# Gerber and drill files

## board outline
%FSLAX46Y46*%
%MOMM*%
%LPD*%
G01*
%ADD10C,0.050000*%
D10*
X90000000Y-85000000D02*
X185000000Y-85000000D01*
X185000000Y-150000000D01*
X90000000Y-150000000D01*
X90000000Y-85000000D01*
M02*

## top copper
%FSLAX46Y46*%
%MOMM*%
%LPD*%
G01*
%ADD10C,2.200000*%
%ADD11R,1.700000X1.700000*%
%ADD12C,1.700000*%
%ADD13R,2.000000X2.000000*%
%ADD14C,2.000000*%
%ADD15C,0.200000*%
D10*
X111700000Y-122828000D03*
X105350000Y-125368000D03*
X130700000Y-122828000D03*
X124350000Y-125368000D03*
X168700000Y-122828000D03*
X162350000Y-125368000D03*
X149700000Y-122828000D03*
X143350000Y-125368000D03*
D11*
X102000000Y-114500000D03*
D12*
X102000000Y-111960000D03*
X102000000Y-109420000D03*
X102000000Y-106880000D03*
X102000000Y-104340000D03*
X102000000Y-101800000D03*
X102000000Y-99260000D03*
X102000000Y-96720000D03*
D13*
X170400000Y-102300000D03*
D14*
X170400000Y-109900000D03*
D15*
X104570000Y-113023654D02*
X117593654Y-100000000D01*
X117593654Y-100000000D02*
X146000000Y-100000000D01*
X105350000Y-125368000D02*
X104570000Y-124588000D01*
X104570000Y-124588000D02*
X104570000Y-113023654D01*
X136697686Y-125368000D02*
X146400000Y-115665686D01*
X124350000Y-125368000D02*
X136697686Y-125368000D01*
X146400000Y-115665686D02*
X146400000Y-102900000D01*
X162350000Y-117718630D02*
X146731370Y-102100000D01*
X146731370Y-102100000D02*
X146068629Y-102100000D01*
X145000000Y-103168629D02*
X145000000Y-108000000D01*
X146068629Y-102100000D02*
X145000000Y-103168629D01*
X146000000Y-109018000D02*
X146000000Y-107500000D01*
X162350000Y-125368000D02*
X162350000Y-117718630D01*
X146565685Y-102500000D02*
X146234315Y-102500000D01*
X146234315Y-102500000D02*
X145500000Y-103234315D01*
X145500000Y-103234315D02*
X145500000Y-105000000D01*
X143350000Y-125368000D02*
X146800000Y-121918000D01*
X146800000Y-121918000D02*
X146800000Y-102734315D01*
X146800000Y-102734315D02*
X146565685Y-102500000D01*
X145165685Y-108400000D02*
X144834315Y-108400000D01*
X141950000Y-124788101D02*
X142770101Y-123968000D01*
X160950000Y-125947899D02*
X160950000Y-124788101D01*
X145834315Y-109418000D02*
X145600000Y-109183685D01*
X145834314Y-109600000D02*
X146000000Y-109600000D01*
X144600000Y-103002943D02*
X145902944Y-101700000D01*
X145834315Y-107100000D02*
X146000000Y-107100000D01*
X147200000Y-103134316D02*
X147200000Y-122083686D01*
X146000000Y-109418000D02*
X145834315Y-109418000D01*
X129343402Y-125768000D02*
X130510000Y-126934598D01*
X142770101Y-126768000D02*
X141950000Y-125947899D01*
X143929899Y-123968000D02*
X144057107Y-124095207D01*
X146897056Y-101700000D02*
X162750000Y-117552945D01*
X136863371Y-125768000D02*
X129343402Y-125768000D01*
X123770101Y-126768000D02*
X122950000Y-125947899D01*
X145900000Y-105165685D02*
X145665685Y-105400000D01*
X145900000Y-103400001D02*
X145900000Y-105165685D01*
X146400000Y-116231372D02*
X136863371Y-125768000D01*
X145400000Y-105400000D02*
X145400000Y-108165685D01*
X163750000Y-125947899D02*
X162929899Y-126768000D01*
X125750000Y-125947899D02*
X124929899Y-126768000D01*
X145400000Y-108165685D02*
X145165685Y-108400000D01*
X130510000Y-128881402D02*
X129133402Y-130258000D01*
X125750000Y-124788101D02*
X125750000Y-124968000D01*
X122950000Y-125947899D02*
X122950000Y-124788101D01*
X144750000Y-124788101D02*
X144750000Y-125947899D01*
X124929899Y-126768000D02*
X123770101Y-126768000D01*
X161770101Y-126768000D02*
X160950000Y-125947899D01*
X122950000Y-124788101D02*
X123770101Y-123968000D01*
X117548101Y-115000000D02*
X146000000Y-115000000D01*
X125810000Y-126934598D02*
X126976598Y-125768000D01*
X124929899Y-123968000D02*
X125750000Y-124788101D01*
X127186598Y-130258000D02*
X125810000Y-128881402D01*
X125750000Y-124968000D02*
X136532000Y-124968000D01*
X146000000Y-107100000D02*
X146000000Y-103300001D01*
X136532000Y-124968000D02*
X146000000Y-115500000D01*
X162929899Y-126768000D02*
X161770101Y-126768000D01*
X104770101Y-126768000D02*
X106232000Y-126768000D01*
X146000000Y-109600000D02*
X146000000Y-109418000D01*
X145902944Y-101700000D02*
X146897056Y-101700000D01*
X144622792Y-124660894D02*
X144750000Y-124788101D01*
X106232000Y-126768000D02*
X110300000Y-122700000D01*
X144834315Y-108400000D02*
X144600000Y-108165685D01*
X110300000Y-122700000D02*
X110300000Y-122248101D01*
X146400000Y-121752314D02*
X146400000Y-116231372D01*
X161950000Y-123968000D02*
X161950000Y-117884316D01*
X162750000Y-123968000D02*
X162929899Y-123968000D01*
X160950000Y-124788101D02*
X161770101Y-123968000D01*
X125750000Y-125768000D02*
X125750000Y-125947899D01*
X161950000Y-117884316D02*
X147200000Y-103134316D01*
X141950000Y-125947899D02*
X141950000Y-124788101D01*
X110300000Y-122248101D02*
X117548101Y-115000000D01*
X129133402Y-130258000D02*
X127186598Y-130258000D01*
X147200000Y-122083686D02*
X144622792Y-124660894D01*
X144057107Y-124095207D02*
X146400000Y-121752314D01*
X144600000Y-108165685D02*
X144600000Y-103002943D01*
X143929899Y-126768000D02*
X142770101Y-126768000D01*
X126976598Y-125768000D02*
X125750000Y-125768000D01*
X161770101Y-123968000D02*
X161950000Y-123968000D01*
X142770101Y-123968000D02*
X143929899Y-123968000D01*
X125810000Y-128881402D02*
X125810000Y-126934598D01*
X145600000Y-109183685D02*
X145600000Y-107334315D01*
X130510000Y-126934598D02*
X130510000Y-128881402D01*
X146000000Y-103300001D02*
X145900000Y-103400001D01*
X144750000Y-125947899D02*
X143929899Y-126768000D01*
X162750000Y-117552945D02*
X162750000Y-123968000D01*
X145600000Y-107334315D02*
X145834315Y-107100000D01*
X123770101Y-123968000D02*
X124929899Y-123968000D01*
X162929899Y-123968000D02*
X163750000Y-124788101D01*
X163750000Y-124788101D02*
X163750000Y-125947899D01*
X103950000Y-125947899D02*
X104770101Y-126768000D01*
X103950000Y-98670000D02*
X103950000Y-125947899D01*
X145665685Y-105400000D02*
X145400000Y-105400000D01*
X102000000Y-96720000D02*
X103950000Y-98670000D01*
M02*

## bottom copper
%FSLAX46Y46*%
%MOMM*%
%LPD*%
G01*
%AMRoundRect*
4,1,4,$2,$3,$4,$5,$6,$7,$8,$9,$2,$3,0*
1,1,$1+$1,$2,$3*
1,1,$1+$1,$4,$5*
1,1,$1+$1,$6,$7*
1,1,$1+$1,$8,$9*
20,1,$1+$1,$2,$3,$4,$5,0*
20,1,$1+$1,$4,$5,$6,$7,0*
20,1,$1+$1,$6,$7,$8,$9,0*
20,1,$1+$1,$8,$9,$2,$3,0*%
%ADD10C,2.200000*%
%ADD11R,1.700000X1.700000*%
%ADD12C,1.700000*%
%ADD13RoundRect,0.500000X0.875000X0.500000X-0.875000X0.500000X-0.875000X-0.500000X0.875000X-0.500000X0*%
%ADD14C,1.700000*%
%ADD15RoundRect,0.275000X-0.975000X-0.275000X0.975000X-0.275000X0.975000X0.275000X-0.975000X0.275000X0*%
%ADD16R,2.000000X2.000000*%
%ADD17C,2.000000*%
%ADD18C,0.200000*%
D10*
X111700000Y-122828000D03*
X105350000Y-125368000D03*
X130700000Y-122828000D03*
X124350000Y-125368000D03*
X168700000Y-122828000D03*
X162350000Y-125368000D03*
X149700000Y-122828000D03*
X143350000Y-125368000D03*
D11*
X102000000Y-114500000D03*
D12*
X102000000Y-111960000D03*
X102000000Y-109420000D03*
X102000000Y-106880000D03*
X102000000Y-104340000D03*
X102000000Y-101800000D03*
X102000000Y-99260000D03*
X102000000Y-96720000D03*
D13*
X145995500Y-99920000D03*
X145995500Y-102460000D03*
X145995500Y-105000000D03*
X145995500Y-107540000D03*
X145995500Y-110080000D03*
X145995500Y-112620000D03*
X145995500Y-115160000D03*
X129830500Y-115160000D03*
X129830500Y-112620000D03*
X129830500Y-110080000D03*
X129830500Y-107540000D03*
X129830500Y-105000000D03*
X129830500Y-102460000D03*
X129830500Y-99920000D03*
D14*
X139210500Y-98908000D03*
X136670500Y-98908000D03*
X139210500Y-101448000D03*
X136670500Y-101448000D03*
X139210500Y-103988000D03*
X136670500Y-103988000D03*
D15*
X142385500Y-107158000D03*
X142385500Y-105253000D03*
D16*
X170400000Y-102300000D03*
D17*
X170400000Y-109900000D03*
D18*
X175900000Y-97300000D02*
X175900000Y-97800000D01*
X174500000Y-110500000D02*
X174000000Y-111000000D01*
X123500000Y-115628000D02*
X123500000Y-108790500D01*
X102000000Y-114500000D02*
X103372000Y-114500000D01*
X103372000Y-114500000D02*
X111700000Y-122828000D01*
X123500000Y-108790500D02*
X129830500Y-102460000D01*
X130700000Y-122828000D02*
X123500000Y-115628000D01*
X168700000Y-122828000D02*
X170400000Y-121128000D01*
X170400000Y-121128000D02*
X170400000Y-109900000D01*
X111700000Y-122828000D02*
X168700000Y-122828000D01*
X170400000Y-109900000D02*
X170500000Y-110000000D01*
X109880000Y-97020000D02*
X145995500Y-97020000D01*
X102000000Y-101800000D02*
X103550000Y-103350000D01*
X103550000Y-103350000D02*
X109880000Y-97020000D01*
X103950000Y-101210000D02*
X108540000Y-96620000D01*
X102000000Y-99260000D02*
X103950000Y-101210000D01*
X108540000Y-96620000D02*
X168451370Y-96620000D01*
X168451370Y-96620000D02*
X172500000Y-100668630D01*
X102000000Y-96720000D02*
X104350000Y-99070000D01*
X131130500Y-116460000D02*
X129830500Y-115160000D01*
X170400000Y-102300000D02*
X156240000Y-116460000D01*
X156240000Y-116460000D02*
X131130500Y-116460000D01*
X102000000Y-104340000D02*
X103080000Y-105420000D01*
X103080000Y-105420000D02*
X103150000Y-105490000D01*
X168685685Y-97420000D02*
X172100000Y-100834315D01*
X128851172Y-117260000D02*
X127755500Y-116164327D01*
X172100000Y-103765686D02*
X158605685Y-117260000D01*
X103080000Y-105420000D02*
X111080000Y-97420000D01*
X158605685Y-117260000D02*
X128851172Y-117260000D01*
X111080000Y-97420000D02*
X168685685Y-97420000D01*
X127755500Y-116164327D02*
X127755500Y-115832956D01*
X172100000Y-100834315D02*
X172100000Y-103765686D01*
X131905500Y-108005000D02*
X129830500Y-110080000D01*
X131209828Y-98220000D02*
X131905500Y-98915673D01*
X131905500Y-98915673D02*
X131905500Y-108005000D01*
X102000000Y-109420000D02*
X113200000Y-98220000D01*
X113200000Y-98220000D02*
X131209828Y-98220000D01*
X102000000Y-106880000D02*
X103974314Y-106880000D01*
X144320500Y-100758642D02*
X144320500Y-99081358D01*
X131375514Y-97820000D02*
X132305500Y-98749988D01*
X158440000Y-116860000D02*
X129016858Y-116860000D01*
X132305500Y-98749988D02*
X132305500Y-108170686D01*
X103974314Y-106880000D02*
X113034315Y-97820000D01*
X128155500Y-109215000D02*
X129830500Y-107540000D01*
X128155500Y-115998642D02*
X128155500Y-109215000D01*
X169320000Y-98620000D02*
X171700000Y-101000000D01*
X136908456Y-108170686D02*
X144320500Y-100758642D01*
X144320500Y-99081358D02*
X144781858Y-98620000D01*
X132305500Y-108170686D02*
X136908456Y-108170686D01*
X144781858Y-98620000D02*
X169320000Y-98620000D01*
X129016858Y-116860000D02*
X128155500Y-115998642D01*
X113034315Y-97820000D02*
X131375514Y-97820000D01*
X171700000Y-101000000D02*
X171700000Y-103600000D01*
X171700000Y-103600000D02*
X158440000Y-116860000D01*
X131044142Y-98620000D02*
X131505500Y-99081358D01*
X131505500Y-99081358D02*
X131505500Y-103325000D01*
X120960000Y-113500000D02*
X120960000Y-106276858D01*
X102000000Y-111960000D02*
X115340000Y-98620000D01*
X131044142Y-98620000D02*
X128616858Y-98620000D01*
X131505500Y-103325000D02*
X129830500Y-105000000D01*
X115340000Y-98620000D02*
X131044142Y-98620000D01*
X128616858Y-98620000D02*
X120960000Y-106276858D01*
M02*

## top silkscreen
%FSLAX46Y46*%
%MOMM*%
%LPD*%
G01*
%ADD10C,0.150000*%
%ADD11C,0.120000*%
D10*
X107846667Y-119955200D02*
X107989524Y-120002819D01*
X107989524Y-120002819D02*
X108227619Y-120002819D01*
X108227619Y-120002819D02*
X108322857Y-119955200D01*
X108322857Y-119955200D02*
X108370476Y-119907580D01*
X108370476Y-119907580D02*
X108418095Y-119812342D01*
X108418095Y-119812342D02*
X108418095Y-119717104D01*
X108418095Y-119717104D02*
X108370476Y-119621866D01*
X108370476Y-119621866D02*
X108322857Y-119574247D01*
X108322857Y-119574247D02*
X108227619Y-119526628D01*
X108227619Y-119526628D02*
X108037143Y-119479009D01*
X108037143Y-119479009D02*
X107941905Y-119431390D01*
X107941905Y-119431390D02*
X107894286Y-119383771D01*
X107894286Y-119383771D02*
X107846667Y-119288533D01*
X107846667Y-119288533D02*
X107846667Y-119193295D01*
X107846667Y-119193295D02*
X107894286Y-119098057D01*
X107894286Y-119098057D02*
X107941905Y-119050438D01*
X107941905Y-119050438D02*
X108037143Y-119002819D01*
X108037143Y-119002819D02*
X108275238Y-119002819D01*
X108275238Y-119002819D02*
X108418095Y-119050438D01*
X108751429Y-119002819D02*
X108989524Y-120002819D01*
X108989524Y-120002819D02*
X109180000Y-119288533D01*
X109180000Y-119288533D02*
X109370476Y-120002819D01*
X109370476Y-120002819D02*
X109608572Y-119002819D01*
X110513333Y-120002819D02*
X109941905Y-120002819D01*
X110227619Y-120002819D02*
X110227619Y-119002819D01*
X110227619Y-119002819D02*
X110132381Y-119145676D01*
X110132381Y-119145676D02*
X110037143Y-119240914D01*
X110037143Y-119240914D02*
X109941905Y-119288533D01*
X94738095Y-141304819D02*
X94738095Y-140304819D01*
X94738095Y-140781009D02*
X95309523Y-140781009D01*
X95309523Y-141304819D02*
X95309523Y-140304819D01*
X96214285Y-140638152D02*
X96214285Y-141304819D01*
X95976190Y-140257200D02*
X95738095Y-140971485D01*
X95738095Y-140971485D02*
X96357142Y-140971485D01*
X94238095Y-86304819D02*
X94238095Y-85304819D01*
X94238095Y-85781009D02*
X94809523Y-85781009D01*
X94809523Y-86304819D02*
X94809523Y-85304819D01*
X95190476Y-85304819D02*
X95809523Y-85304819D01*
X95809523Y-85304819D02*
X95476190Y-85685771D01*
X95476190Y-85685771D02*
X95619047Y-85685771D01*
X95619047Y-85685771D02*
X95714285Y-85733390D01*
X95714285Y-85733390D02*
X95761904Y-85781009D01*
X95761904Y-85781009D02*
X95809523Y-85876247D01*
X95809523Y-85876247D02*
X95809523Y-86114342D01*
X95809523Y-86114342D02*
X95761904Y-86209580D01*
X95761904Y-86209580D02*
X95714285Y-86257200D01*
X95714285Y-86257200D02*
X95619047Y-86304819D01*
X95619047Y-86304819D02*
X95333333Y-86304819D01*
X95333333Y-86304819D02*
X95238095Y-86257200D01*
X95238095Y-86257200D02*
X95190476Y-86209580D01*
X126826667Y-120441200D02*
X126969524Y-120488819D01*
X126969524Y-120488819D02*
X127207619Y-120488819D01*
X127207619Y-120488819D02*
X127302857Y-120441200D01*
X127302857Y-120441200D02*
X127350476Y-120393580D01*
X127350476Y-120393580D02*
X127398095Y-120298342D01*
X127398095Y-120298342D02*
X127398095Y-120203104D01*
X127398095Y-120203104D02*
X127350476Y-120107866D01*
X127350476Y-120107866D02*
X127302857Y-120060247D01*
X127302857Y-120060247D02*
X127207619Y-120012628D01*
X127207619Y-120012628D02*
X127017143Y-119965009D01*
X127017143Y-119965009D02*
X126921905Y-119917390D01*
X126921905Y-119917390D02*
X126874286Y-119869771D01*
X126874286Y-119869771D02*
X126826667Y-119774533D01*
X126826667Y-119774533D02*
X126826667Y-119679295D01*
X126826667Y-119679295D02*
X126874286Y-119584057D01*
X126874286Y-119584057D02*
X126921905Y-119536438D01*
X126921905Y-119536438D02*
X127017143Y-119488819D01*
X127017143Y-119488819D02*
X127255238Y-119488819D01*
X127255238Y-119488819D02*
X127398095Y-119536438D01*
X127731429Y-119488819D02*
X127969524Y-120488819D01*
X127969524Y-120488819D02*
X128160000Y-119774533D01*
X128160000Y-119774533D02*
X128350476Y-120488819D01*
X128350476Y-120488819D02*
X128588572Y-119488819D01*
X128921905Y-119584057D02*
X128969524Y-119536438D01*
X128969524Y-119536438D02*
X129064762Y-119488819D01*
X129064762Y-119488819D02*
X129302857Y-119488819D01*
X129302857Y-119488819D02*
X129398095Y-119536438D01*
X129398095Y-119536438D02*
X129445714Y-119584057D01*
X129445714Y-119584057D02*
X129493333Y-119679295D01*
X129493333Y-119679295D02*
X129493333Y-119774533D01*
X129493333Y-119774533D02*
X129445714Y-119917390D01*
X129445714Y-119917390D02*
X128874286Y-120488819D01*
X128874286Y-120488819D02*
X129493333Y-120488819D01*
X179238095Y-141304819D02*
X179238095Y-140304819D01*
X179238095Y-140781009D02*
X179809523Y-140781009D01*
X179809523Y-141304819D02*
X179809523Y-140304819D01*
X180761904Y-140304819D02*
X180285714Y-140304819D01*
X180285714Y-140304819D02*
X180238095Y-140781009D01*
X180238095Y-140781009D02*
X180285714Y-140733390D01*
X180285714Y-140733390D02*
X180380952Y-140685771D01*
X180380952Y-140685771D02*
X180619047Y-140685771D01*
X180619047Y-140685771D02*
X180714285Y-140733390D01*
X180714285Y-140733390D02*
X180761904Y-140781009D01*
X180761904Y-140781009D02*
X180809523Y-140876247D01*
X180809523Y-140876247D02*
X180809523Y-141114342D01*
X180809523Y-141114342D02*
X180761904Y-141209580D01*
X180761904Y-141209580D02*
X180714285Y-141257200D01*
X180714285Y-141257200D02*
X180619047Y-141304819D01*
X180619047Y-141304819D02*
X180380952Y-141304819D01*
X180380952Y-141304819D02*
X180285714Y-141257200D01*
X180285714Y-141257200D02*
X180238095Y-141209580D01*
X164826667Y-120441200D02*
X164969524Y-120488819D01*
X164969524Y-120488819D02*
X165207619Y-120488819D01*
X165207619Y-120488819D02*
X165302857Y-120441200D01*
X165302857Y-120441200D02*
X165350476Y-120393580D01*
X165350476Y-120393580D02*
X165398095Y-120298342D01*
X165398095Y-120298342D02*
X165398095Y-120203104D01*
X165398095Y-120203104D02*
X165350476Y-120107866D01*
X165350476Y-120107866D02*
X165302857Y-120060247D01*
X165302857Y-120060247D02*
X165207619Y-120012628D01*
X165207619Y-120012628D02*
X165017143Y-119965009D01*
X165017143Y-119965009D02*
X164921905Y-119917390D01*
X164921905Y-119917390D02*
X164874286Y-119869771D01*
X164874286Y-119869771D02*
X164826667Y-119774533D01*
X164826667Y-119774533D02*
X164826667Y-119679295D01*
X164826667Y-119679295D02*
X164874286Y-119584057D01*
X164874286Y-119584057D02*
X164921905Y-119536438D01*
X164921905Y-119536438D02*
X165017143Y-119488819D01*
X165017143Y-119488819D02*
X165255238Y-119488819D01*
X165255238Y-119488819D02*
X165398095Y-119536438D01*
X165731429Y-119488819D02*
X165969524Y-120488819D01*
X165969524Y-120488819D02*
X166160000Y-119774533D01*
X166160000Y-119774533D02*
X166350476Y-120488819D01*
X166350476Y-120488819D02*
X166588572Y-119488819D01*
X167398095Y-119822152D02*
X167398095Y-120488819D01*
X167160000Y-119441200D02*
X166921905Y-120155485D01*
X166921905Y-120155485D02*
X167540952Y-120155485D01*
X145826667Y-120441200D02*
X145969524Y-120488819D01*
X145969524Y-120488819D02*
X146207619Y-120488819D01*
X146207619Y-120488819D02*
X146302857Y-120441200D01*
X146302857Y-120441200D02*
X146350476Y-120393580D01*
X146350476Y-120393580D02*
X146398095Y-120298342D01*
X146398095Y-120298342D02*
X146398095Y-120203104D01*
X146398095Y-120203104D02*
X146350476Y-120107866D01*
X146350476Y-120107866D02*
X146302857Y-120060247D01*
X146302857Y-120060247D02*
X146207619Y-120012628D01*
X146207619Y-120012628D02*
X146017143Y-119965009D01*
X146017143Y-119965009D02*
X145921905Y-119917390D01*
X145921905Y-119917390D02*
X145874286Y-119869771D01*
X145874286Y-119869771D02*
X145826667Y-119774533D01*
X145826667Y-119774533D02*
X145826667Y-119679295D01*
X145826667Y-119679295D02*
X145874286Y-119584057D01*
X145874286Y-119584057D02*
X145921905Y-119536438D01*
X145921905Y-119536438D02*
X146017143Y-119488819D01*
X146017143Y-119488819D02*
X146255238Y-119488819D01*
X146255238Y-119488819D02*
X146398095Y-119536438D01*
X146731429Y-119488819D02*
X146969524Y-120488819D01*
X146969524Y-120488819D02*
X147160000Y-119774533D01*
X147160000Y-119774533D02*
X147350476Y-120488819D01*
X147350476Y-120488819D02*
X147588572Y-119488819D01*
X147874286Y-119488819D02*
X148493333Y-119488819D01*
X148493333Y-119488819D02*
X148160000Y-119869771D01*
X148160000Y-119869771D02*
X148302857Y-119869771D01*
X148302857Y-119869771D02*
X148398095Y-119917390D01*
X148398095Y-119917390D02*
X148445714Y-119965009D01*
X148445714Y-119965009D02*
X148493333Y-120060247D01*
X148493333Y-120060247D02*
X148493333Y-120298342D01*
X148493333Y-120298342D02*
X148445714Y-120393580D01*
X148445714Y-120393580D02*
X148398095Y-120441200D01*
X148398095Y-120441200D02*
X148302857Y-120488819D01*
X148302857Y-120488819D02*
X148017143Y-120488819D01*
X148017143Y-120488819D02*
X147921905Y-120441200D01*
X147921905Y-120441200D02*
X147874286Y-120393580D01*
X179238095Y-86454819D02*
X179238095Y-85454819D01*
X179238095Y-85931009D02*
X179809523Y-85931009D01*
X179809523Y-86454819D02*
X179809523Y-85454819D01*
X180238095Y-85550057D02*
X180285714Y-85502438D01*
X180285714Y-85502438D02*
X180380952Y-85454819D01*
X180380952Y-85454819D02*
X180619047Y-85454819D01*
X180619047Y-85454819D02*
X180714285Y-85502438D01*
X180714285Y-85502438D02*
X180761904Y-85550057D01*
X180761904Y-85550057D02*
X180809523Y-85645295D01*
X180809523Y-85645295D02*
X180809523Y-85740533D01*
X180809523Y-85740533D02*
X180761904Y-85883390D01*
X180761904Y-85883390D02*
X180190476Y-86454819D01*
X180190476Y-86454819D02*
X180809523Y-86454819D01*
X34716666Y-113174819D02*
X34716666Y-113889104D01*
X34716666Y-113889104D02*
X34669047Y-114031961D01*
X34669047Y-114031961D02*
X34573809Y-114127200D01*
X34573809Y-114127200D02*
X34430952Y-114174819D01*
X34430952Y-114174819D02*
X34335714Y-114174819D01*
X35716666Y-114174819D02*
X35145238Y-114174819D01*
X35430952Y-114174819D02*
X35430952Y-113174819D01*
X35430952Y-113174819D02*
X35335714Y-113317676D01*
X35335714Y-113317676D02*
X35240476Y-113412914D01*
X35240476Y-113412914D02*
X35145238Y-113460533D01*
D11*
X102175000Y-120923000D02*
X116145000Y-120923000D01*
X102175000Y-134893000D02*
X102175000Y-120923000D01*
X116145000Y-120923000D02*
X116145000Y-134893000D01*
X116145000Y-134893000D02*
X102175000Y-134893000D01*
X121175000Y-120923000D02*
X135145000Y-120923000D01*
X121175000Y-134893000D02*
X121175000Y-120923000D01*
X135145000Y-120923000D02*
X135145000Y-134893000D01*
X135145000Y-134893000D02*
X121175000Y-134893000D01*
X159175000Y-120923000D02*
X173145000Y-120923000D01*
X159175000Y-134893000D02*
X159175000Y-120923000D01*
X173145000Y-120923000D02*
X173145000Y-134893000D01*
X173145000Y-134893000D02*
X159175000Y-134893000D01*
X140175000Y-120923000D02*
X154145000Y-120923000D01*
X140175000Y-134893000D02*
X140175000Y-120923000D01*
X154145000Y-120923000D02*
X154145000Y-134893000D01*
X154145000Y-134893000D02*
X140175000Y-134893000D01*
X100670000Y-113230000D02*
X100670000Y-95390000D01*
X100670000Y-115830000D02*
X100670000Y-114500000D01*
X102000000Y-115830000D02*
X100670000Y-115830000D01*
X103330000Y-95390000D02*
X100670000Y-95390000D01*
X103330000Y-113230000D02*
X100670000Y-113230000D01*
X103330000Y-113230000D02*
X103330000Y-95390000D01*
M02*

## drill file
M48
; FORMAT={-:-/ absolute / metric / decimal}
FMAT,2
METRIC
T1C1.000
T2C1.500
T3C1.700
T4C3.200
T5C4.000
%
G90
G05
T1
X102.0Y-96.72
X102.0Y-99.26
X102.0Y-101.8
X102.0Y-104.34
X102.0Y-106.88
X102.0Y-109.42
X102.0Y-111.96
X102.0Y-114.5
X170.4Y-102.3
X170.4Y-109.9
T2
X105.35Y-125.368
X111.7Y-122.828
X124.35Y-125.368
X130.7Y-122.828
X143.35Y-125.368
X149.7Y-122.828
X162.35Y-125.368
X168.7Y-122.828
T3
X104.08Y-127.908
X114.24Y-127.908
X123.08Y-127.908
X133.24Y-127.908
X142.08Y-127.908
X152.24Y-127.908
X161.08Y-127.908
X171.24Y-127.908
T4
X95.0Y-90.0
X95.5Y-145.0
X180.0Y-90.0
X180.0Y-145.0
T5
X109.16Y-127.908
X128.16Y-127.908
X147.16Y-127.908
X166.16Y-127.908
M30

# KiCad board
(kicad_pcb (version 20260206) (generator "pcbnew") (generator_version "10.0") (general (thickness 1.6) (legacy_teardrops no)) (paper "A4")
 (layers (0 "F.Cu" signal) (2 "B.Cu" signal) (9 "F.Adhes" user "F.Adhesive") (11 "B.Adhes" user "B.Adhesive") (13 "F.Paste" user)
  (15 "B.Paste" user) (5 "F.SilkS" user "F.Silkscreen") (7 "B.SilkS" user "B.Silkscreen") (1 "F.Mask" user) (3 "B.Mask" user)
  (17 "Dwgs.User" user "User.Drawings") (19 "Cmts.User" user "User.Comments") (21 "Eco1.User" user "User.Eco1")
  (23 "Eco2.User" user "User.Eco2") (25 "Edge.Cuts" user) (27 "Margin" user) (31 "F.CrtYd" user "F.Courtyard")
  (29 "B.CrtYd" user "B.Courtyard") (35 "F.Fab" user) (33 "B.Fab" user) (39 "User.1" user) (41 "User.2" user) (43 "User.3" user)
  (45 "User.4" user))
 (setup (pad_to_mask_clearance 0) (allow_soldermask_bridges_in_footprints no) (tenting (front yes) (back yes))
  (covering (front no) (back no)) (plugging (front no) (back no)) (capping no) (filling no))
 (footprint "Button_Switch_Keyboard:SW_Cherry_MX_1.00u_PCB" (layer "F.Cu") (at 111.7 122.828)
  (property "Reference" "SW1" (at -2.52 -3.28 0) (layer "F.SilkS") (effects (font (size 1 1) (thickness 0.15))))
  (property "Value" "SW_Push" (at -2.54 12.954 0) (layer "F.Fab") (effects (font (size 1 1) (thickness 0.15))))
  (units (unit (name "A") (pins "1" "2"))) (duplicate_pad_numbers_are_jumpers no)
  (fp_line (start -9.525 -1.905) (end 4.445 -1.905) (stroke (width 0.12) (type solid)) (layer "F.SilkS"))
  (fp_line (start -9.525 12.065) (end -9.525 -1.905) (stroke (width 0.12) (type solid)) (layer "F.SilkS"))
  (fp_line (start 4.445 -1.905) (end 4.445 12.065) (stroke (width 0.12) (type solid)) (layer "F.SilkS"))
  (fp_line (start 4.445 12.065) (end -9.525 12.065) (stroke (width 0.12) (type solid)) (layer "F.SilkS"))
  (pad "" np_thru_hole circle (at -7.62 5.08) (size 1.7 1.7) (drill 1.7) (layers "*.Cu" "*.Mask"))
  (pad "" np_thru_hole circle (at -2.54 5.08) (size 4 4) (drill 4) (layers "*.Cu" "*.Mask"))
  (pad "" np_thru_hole circle (at 2.54 5.08) (size 1.7 1.7) (drill 1.7) (layers "*.Cu" "*.Mask"))
  (pad "1" thru_hole circle (at 0 0) (size 2.2 2.2) (drill 1.5) (layers "*.Cu" "*.Mask") (remove_unused_layers no) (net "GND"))
  (pad "2" thru_hole circle (at -6.35 2.54) (size 2.2 2.2) (drill 1.5) (layers "*.Cu" "*.Mask") (remove_unused_layers no)
   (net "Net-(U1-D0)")))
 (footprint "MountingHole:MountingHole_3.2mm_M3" (layer "F.Cu") (at 95.5 145)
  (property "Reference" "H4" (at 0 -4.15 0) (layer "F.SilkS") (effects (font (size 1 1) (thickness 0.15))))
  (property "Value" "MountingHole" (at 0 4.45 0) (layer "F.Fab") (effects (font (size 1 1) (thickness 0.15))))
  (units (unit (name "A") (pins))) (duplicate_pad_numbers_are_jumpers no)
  (pad "" np_thru_hole circle (at 0 0) (size 3.2 3.2) (drill 3.2) (layers "*.Cu" "*.Mask")))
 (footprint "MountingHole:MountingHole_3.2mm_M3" (layer "F.Cu") (at 95 90)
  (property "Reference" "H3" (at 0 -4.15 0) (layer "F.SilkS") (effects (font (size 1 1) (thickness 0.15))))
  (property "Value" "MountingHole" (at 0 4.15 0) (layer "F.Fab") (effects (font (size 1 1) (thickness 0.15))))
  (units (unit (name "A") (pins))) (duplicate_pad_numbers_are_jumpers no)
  (pad "" np_thru_hole circle (at 0 0) (size 3.2 3.2) (drill 3.2) (layers "*.Cu" "*.Mask")))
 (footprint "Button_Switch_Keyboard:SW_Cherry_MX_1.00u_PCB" (layer "F.Cu") (at 130.7 122.828)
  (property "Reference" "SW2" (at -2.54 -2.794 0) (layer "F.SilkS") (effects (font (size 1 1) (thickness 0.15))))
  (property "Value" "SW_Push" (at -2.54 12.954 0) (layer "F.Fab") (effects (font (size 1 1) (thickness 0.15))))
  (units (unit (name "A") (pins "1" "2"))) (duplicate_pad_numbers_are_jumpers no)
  (fp_line (start -9.525 -1.905) (end 4.445 -1.905) (stroke (width 0.12) (type solid)) (layer "F.SilkS"))
  (fp_line (start -9.525 12.065) (end -9.525 -1.905) (stroke (width 0.12) (type solid)) (layer "F.SilkS"))
  (fp_line (start 4.445 -1.905) (end 4.445 12.065) (stroke (width 0.12) (type solid)) (layer "F.SilkS"))
  (fp_line (start 4.445 12.065) (end -9.525 12.065) (stroke (width 0.12) (type solid)) (layer "F.SilkS"))
  (pad "" np_thru_hole circle (at -7.62 5.08) (size 1.7 1.7) (drill 1.7) (layers "*.Cu" "*.Mask"))
  (pad "" np_thru_hole circle (at -2.54 5.08) (size 4 4) (drill 4) (layers "*.Cu" "*.Mask"))
  (pad "" np_thru_hole circle (at 2.54 5.08) (size 1.7 1.7) (drill 1.7) (layers "*.Cu" "*.Mask"))
  (pad "1" thru_hole circle (at 0 0) (size 2.2 2.2) (drill 1.5) (layers "*.Cu" "*.Mask") (remove_unused_layers no) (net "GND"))
  (pad "2" thru_hole circle (at -6.35 2.54) (size 2.2 2.2) (drill 1.5) (layers "*.Cu" "*.Mask") (remove_unused_layers no)
   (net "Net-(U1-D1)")))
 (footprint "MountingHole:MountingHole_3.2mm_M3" (layer "F.Cu") (at 180 145)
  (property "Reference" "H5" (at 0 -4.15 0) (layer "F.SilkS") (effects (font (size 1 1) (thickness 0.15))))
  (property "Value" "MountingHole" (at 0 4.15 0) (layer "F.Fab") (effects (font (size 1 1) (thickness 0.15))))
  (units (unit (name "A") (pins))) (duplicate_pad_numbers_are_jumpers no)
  (pad "" np_thru_hole circle (at 0 0) (size 3.2 3.2) (drill 3.2) (layers "*.Cu" "*.Mask")))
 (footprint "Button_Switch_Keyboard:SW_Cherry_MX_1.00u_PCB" (layer "F.Cu") (at 168.7 122.828)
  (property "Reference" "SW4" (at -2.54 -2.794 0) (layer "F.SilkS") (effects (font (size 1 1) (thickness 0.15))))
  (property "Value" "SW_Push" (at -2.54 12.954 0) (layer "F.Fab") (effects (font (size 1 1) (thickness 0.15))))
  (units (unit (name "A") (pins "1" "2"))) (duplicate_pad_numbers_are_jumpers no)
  (fp_line (start -9.525 -1.905) (end 4.445 -1.905) (stroke (width 0.12) (type solid)) (layer "F.SilkS"))
  (fp_line (start -9.525 12.065) (end -9.525 -1.905) (stroke (width 0.12) (type solid)) (layer "F.SilkS"))
  (fp_line (start 4.445 -1.905) (end 4.445 12.065) (stroke (width 0.12) (type solid)) (layer "F.SilkS"))
  (fp_line (start 4.445 12.065) (end -9.525 12.065) (stroke (width 0.12) (type solid)) (layer "F.SilkS"))
  (pad "" np_thru_hole circle (at -7.62 5.08) (size 1.7 1.7) (drill 1.7) (layers "*.Cu" "*.Mask"))
  (pad "" np_thru_hole circle (at -2.54 5.08) (size 4 4) (drill 4) (layers "*.Cu" "*.Mask"))
  (pad "" np_thru_hole circle (at 2.54 5.08) (size 1.7 1.7) (drill 1.7) (layers "*.Cu" "*.Mask"))
  (pad "1" thru_hole circle (at 0 0) (size 2.2 2.2) (drill 1.5) (layers "*.Cu" "*.Mask") (remove_unused_layers no) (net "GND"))
  (pad "2" thru_hole circle (at -6.35 2.54) (size 2.2 2.2) (drill 1.5) (layers "*.Cu" "*.Mask") (remove_unused_layers no)
   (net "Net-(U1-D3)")))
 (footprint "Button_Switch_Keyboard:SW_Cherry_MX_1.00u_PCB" (layer "F.Cu") (at 149.7 122.828)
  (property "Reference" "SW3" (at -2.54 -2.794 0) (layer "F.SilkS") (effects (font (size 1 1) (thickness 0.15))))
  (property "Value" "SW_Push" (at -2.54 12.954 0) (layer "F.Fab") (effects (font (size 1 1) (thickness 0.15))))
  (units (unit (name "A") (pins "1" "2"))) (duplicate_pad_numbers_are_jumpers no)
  (fp_line (start -9.525 -1.905) (end 4.445 -1.905) (stroke (width 0.12) (type solid)) (layer "F.SilkS"))
  (fp_line (start -9.525 12.065) (end -9.525 -1.905) (stroke (width 0.12) (type solid)) (layer "F.SilkS"))
  (fp_line (start 4.445 -1.905) (end 4.445 12.065) (stroke (width 0.12) (type solid)) (layer "F.SilkS"))
  (fp_line (start 4.445 12.065) (end -9.525 12.065) (stroke (width 0.12) (type solid)) (layer "F.SilkS"))
  (pad "" np_thru_hole circle (at -7.62 5.08) (size 1.7 1.7) (drill 1.7) (layers "*.Cu" "*.Mask"))
  (pad "" np_thru_hole circle (at -2.54 5.08) (size 4 4) (drill 4) (layers "*.Cu" "*.Mask"))
  (pad "" np_thru_hole circle (at 2.54 5.08) (size 1.7 1.7) (drill 1.7) (layers "*.Cu" "*.Mask"))
  (pad "1" thru_hole circle (at 0 0) (size 2.2 2.2) (drill 1.5) (layers "*.Cu" "*.Mask") (remove_unused_layers no) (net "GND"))
  (pad "2" thru_hole circle (at -6.35 2.54) (size 2.2 2.2) (drill 1.5) (layers "*.Cu" "*.Mask") (remove_unused_layers no)
   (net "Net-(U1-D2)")))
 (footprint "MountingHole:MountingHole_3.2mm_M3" (layer "F.Cu") (at 180 90)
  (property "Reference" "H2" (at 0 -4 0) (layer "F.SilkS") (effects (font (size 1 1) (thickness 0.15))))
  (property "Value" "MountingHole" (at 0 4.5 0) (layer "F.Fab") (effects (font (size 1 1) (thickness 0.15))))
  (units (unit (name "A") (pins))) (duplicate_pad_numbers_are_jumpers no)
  (pad "" np_thru_hole circle (at 0 0) (size 3.2 3.2) (drill 3.2) (layers "*.Cu" "*.Mask")))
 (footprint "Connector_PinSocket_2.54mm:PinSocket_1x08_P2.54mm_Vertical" (layer "F.Cu") (at 102 114.5 180)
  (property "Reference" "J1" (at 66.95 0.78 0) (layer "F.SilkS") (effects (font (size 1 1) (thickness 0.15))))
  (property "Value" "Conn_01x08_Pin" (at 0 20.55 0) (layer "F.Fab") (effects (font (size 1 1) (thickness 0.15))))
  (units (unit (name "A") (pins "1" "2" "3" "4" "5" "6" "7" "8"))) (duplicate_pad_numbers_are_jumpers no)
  (fp_line (start 1.33 1.27) (end 1.33 19.11) (stroke (width 0.12) (type solid)) (layer "F.SilkS"))
  (fp_line (start 1.33 -1.33) (end 1.33 0) (stroke (width 0.12) (type solid)) (layer "F.SilkS"))
  (fp_line (start 0 -1.33) (end 1.33 -1.33) (stroke (width 0.12) (type solid)) (layer "F.SilkS"))
  (fp_line (start -1.33 19.11) (end 1.33 19.11) (stroke (width 0.12) (type solid)) (layer "F.SilkS"))
  (fp_line (start -1.33 1.27) (end 1.33 1.27) (stroke (width 0.12) (type solid)) (layer "F.SilkS"))
  (fp_line (start -1.33 1.27) (end -1.33 19.11) (stroke (width 0.12) (type solid)) (layer "F.SilkS"))
  (pad "1" thru_hole rect (at 0 0 180) (size 1.7 1.7) (drill 1) (layers "*.Cu" "*.Mask") (remove_unused_layers no) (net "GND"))
  (pad "2" thru_hole circle (at 0 2.54 180) (size 1.7 1.7) (drill 1) (layers "*.Cu" "*.Mask") (remove_unused_layers no) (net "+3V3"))
  (pad "3" thru_hole circle (at 0 5.08 180) (size 1.7 1.7) (drill 1) (layers "*.Cu" "*.Mask") (remove_unused_layers no) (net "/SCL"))
  (pad "4" thru_hole circle (at 0 7.62 180) (size 1.7 1.7) (drill 1) (layers "*.Cu" "*.Mask") (remove_unused_layers no) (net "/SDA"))
  (pad "5" thru_hole circle (at 0 10.16 180) (size 1.7 1.7) (drill 1) (layers "*.Cu" "*.Mask") (remove_unused_layers no) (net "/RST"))
  (pad "6" thru_hole circle (at 0 12.7 180) (size 1.7 1.7) (drill 1) (layers "*.Cu" "*.Mask") (remove_unused_layers no) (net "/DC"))
  (pad "7" thru_hole circle (at 0 15.24 180) (size 1.7 1.7) (drill 1) (layers "*.Cu" "*.Mask") (remove_unused_layers no) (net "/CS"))
  (pad "8" thru_hole circle (at 0 17.78 180) (size 1.7 1.7) (drill 1) (layers "*.Cu" "*.Mask") (remove_unused_layers no) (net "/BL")))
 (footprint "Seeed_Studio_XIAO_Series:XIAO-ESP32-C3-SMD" (layer "B.Cu") (at 146.8305 118.04 180)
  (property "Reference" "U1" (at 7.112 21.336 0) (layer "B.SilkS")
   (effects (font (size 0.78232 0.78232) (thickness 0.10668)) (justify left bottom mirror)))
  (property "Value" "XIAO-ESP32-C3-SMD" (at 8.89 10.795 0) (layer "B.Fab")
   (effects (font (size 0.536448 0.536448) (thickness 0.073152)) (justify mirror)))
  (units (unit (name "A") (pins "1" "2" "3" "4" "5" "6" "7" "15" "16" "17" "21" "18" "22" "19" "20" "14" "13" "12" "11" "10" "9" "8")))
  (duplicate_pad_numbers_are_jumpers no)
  (pad "1" smd roundrect (at 0.835 18.12 180) (size 2.75 2) (layers "B.Cu" "B.Mask" "B.Paste") (roundrect_rratio 0.25) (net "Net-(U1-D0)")
   (solder_mask_margin 0.0508) (thermal_bridge_angle 45))
  (pad "2" smd roundrect (at 0.835 15.58 180) (size 2.75 2) (layers "B.Cu" "B.Mask" "B.Paste") (roundrect_rratio 0.25) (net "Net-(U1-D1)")
   (solder_mask_margin 0.0508) (thermal_bridge_angle 45))
  (pad "3" smd roundrect (at 0.835 13.04 180) (size 2.75 2) (layers "B.Cu" "B.Mask" "B.Paste") (roundrect_rratio 0.25) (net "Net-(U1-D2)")
   (solder_mask_margin 0.0508) (thermal_bridge_angle 45))
  (pad "4" smd roundrect (at 0.835 10.5 180) (size 2.75 2) (layers "B.Cu" "B.Mask" "B.Paste") (roundrect_rratio 0.25) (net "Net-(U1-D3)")
   (solder_mask_margin 0.0508) (thermal_bridge_angle 45))
  (pad "5" smd roundrect (at 0.835 7.96 180) (size 2.75 2) (layers "B.Cu" "B.Mask" "B.Paste") (roundrect_rratio 0.25) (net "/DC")
   (solder_mask_margin 0.0508) (thermal_bridge_angle 45))
  (pad "6" smd roundrect (at 0.835 5.42 180) (size 2.75 2) (layers "B.Cu" "B.Mask" "B.Paste") (roundrect_rratio 0.25) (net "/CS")
   (solder_mask_margin 0.0508) (thermal_bridge_angle 45))
  (pad "7" smd roundrect (at 0.835 2.88 180) (size 2.75 2) (layers "B.Cu" "B.Mask" "B.Paste") (roundrect_rratio 0.25) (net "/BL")
   (solder_mask_margin 0.0508) (thermal_bridge_angle 45))
  (pad "8" smd roundrect (at 17 2.88 180) (size 2.75 2) (layers "B.Cu" "B.Mask" "B.Paste") (roundrect_rratio 0.25) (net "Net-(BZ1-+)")
   (solder_mask_margin 0.0508) (thermal_bridge_angle 45))
  (pad "9" smd roundrect (at 17 5.42 180) (size 2.75 2) (layers "B.Cu" "B.Mask" "B.Paste") (roundrect_rratio 0.25) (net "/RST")
   (solder_mask_margin 0.0508) (thermal_bridge_angle 45))
  (pad "10" smd roundrect (at 17 7.96 180) (size 2.75 2) (layers "B.Cu" "B.Mask" "B.Paste") (roundrect_rratio 0.25) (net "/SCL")
   (solder_mask_margin 0.0508) (thermal_bridge_angle 45))
  (pad "11" smd roundrect (at 17 10.5 180) (size 2.75 2) (layers "B.Cu" "B.Mask" "B.Paste") (roundrect_rratio 0.25) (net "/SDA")
   (solder_mask_margin 0.0508) (thermal_bridge_angle 45))
  (pad "12" smd roundrect (at 17 13.04 180) (size 2.75 2) (layers "B.Cu" "B.Mask" "B.Paste") (roundrect_rratio 0.25) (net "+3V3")
   (solder_mask_margin 0.0508) (thermal_bridge_angle 45))
  (pad "13" smd roundrect (at 17 15.58 180) (size 2.75 2) (layers "B.Cu" "B.Mask" "B.Paste") (roundrect_rratio 0.25) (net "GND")
   (solder_mask_margin 0.0508) (thermal_bridge_angle 45))
  (pad "14" smd roundrect (at 17 18.12 180) (size 2.75 2) (layers "B.Cu" "B.Mask" "B.Paste") (roundrect_rratio 0.25)
   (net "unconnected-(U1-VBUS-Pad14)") (solder_mask_margin 0.0508) (thermal_bridge_angle 45))
  (pad "15" smd circle (at 7.62 19.132 180) (size 1.7 1.7) (layers "B.Cu" "B.Mask" "B.Paste") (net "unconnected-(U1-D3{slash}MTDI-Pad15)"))
  (pad "16" smd circle (at 10.16 19.132 180) (size 1.7 1.7) (layers "B.Cu" "B.Mask" "B.Paste") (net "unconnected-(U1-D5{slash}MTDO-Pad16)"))
  (pad "17" smd circle (at 7.62 16.592 180) (size 1.7 1.7) (layers "B.Cu" "B.Mask" "B.Paste") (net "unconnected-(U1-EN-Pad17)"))
  (pad "18" smd circle (at 10.16 16.592 180) (size 1.7 1.7) (layers "B.Cu" "B.Mask" "B.Paste") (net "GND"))
  (pad "19" smd circle (at 7.62 14.052 180) (size 1.7 1.7) (layers "B.Cu" "B.Mask" "B.Paste") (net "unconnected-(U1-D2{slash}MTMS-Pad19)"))
  (pad "20" smd circle (at 10.16 14.052 180) (size 1.7 1.7) (layers "B.Cu" "B.Mask" "B.Paste") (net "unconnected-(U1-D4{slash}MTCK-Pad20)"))
  (pad "21" smd roundrect (at 4.445 10.882) (size 2.5 1.1) (layers "B.Cu" "B.Mask" "B.Paste") (roundrect_rratio 0.25)
   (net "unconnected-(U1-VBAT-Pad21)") (thermal_bridge_angle 45))
  (pad "22" smd roundrect (at 4.445 12.787) (size 2.5 1.1) (layers "B.Cu" "B.Mask" "B.Paste") (roundrect_rratio 0.25) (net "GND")
   (thermal_bridge_angle 45)))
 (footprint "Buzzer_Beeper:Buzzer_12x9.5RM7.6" (layer "B.Cu") (at 170.4 102.3 -90)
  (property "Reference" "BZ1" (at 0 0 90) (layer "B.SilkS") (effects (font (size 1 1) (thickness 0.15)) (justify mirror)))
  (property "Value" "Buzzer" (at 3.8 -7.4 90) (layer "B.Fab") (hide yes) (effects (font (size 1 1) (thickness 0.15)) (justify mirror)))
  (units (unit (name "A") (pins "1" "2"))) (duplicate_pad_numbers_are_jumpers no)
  (pad "1" thru_hole rect (at 0 0 270) (size 2 2) (drill 1) (layers "*.Cu" "*.Mask") (remove_unused_layers no) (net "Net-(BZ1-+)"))
  (pad "2" thru_hole circle (at 7.6 0 270) (size 2 2) (drill 1) (layers "*.Cu" "*.Mask") (remove_unused_layers no) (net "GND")))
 (gr_rect (start 90 85) (end 185 150) (stroke (width 0.05) (type default)) (fill no) (layer "Edge.Cuts"))
 (segment (start 175.9 97.3) (end 175.9 97.8) (width 0.2) (layer "B.Cu") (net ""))
 (segment (start 174.5 110.5) (end 174 111) (width 0.2) (layer "B.Cu") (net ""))
 (segment (start 123.5 115.628) (end 123.5 108.7905) (width 0.2) (layer "B.Cu") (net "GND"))
 (segment (start 102 114.5) (end 103.372 114.5) (width 0.2) (layer "B.Cu") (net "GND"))
 (segment (start 103.372 114.5) (end 111.7 122.828) (width 0.2) (layer "B.Cu") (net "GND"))
 (segment (start 123.5 108.7905) (end 129.8305 102.46) (width 0.2) (layer "B.Cu") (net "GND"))
 (segment (start 130.7 122.828) (end 123.5 115.628) (width 0.2) (layer "B.Cu") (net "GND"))
 (segment (start 168.7 122.828) (end 170.4 121.128) (width 0.2) (layer "B.Cu") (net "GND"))
 (segment (start 170.4 121.128) (end 170.4 109.9) (width 0.2) (layer "B.Cu") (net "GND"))
 (segment (start 111.7 122.828) (end 168.7 122.828) (width 0.2) (layer "B.Cu") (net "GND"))
 (segment (start 170.4 109.9) (end 170.5 110) (width 0.2) (layer "B.Cu") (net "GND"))
 (segment (start 104.57 113.023654) (end 117.593654 100) (width 0.2) (layer "F.Cu") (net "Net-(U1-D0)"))
 (segment (start 117.593654 100) (end 146 100) (width 0.2) (layer "F.Cu") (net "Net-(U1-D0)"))
 (segment (start 105.35 125.368) (end 104.57 124.588) (width 0.2) (layer "F.Cu") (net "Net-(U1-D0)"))
 (segment (start 104.57 124.588) (end 104.57 113.023654) (width 0.2) (layer "F.Cu") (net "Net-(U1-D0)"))
 (segment (start 136.697686 125.368) (end 146.4 115.665686) (width 0.2) (layer "F.Cu") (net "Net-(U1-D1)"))
 (segment (start 124.35 125.368) (end 136.697686 125.368) (width 0.2) (layer "F.Cu") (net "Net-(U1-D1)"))
 (segment (start 146.4 115.665686) (end 146.4 102.9) (width 0.2) (layer "F.Cu") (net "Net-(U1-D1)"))
 (segment (start 162.35 117.71863) (end 146.73137 102.1) (width 0.2) (layer "F.Cu") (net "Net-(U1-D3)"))
 (segment (start 146.73137 102.1) (end 146.068629 102.1) (width 0.2) (layer "F.Cu") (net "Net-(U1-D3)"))
 (segment (start 145 103.168629) (end 145 108) (width 0.2) (layer "F.Cu") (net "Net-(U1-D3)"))
 (segment (start 146.068629 102.1) (end 145 103.168629) (width 0.2) (layer "F.Cu") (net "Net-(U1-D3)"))
 (segment (start 146 109.018) (end 146 107.5) (width 0.2) (layer "F.Cu") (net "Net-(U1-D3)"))
 (segment (start 162.35 125.368) (end 162.35 117.71863) (width 0.2) (layer "F.Cu") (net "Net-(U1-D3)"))
 (segment (start 146.565685 102.5) (end 146.234315 102.5) (width 0.2) (layer "F.Cu") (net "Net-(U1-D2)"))
 (segment (start 146.234315 102.5) (end 145.5 103.234315) (width 0.2) (layer "F.Cu") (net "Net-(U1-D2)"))
 (segment (start 145.5 103.234315) (end 145.5 105) (width 0.2) (layer "F.Cu") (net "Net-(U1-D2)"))
 (segment (start 143.35 125.368) (end 146.8 121.918) (width 0.2) (layer "F.Cu") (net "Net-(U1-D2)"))
 (segment (start 146.8 121.918) (end 146.8 102.734315) (width 0.2) (layer "F.Cu") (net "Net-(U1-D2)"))
 (segment (start 146.8 102.734315) (end 146.565685 102.5) (width 0.2) (layer "F.Cu") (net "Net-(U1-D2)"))
 (segment (start 109.88 97.02) (end 145.9955 97.02) (width 0.2) (layer "B.Cu") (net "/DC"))
 (segment (start 102 101.8) (end 103.55 103.35) (width 0.2) (layer "B.Cu") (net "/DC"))
 (segment (start 103.55 103.35) (end 109.88 97.02) (width 0.2) (layer "B.Cu") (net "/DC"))
 (segment (start 103.95 101.21) (end 108.54 96.62) (width 0.2) (layer "B.Cu") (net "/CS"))
 (segment (start 102 99.26) (end 103.95 101.21) (width 0.2) (layer "B.Cu") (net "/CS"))
 (segment (start 108.54 96.62) (end 168.45137 96.62) (width 0.2) (layer "B.Cu") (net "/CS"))
 (segment (start 168.45137 96.62) (end 172.5 100.66863) (width 0.2) (layer "B.Cu") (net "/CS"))
 (segment (start 145.165685 108.4) (end 144.834315 108.4) (width 0.2) (layer "F.Cu") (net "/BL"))
 (segment (start 141.95 124.788101) (end 142.770101 123.968) (width 0.2) (layer "F.Cu") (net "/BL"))
 (segment (start 160.95 125.947899) (end 160.95 124.788101) (width 0.2) (layer "F.Cu") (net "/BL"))
 (segment (start 145.834315 109.418) (end 145.6 109.183685) (width 0.2) (layer "F.Cu") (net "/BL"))
 (segment (start 145.834314 109.6) (end 146 109.6) (width 0.2) (layer "F.Cu") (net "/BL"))
 (segment (start 144.6 103.002943) (end 145.902944 101.7) (width 0.2) (layer "F.Cu") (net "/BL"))
 (segment (start 145.834315 107.1) (end 146 107.1) (width 0.2) (layer "F.Cu") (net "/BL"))
 (segment (start 147.2 103.134316) (end 147.2 122.083686) (width 0.2) (layer "F.Cu") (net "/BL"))
 (segment (start 146 109.418) (end 145.834315 109.418) (width 0.2) (layer "F.Cu") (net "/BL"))
 (segment (start 129.343402 125.768) (end 130.51 126.934598) (width 0.2) (layer "F.Cu") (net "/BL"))
 (segment (start 142.770101 126.768) (end 141.95 125.947899) (width 0.2) (layer "F.Cu") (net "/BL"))
 (segment (start 143.929899 123.968) (end 144.057107 124.095207) (width 0.2) (layer "F.Cu") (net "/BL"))
 (segment (start 146.897056 101.7) (end 162.75 117.552945) (width 0.2) (layer "F.Cu") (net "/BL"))
 (segment (start 136.863371 125.768) (end 129.343402 125.768) (width 0.2) (layer "F.Cu") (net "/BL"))
 (segment (start 123.770101 126.768) (end 122.95 125.947899) (width 0.2) (layer "F.Cu") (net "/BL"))
 (segment (start 145.9 105.165685) (end 145.665685 105.4) (width 0.2) (layer "F.Cu") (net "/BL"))
 (segment (start 145.9 103.400001) (end 145.9 105.165685) (width 0.2) (layer "F.Cu") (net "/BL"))
 (segment (start 146.4 116.231372) (end 136.863371 125.768) (width 0.2) (layer "F.Cu") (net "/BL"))
 (segment (start 145.4 105.4) (end 145.4 108.165685) (width 0.2) (layer "F.Cu") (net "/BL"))
 (segment (start 163.75 125.947899) (end 162.929899 126.768) (width 0.2) (layer "F.Cu") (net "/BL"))
 (segment (start 125.75 125.947899) (end 124.929899 126.768) (width 0.2) (layer "F.Cu") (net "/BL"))
 (segment (start 145.4 108.165685) (end 145.165685 108.4) (width 0.2) (layer "F.Cu") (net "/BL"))
 (segment (start 130.51 128.881402) (end 129.133402 130.258) (width 0.2) (layer "F.Cu") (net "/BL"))
 (segment (start 125.75 124.788101) (end 125.75 124.968) (width 0.2) (layer "F.Cu") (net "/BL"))
 (segment (start 122.95 125.947899) (end 122.95 124.788101) (width 0.2) (layer "F.Cu") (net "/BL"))
 (segment (start 144.75 124.788101) (end 144.75 125.947899) (width 0.2) (layer "F.Cu") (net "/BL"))
 (segment (start 124.929899 126.768) (end 123.770101 126.768) (width 0.2) (layer "F.Cu") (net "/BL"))
 (segment (start 161.770101 126.768) (end 160.95 125.947899) (width 0.2) (layer "F.Cu") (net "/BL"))
 (segment (start 122.95 124.788101) (end 123.770101 123.968) (width 0.2) (layer "F.Cu") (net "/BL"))
 (segment (start 117.548101 115) (end 146 115) (width 0.2) (layer "F.Cu") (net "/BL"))
 (segment (start 125.81 126.934598) (end 126.976598 125.768) (width 0.2) (layer "F.Cu") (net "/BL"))
 (segment (start 124.929899 123.968) (end 125.75 124.788101) (width 0.2) (layer "F.Cu") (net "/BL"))
 (segment (start 127.186598 130.258) (end 125.81 128.881402) (width 0.2) (layer "F.Cu") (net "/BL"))
 (segment (start 125.75 124.968) (end 136.532 124.968) (width 0.2) (layer "F.Cu") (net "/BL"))
 (segment (start 146 107.1) (end 146 103.300001) (width 0.2) (layer "F.Cu") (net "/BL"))
 (segment (start 136.532 124.968) (end 146 115.5) (width 0.2) (layer "F.Cu") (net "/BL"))
 (segment (start 162.929899 126.768) (end 161.770101 126.768) (width 0.2) (layer "F.Cu") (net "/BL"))
 (segment (start 104.770101 126.768) (end 106.232 126.768) (width 0.2) (layer "F.Cu") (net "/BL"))
 (segment (start 146 109.6) (end 146 109.418) (width 0.2) (layer "F.Cu") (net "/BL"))
 (segment (start 145.902944 101.7) (end 146.897056 101.7) (width 0.2) (layer "F.Cu") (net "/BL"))
 (segment (start 144.622792 124.660894) (end 144.75 124.788101) (width 0.2) (layer "F.Cu") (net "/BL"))
 (segment (start 106.232 126.768) (end 110.3 122.7) (width 0.2) (layer "F.Cu") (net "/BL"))
 (segment (start 144.834315 108.4) (end 144.6 108.165685) (width 0.2) (layer "F.Cu") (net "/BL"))
 (segment (start 110.3 122.7) (end 110.3 122.248101) (width 0.2) (layer "F.Cu") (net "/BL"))
 (segment (start 146.4 121.752314) (end 146.4 116.231372) (width 0.2) (layer "F.Cu") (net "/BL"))
 (segment (start 161.95 123.968) (end 161.95 117.884316) (width 0.2) (layer "F.Cu") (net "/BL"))
 (segment (start 162.75 123.968) (end 162.929899 123.968) (width 0.2) (layer "F.Cu") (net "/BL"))
 (segment (start 160.95 124.788101) (end 161.770101 123.968) (width 0.2) (layer "F.Cu") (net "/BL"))
 (segment (start 125.75 125.768) (end 125.75 125.947899) (width 0.2) (layer "F.Cu") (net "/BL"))
 (segment (start 161.95 117.884316) (end 147.2 103.134316) (width 0.2) (layer "F.Cu") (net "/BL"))
 (segment (start 141.95 125.947899) (end 141.95 124.788101) (width 0.2) (layer "F.Cu") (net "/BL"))
 (segment (start 110.3 122.248101) (end 117.548101 115) (width 0.2) (layer "F.Cu") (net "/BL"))
 (segment (start 129.133402 130.258) (end 127.186598 130.258) (width 0.2) (layer "F.Cu") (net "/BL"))
 (segment (start 147.2 122.083686) (end 144.622792 124.660894) (width 0.2) (layer "F.Cu") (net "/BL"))
 (segment (start 144.057107 124.095207) (end 146.4 121.752314) (width 0.2) (layer "F.Cu") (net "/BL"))
 (segment (start 144.6 108.165685) (end 144.6 103.002943) (width 0.2) (layer "F.Cu") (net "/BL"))
 (segment (start 143.929899 126.768) (end 142.770101 126.768) (width 0.2) (layer "F.Cu") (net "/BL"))
 (segment (start 126.976598 125.768) (end 125.75 125.768) (width 0.2) (layer "F.Cu") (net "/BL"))
 (segment (start 161.770101 123.968) (end 161.95 123.968) (width 0.2) (layer "F.Cu") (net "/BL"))
 (segment (start 142.770101 123.968) (end 143.929899 123.968) (width 0.2) (layer "F.Cu") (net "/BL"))
 (segment (start 125.81 128.881402) (end 125.81 126.934598) (width 0.2) (layer "F.Cu") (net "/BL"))
 (segment (start 145.6 109.183685) (end 145.6 107.334315) (width 0.2) (layer "F.Cu") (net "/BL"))
 (segment (start 130.51 126.934598) (end 130.51 128.881402) (width 0.2) (layer "F.Cu") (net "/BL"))
 (segment (start 146 103.300001) (end 145.9 103.400001) (width 0.2) (layer "F.Cu") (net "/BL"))
 (segment (start 144.75 125.947899) (end 143.929899 126.768) (width 0.2) (layer "F.Cu") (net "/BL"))
 (segment (start 162.75 117.552945) (end 162.75 123.968) (width 0.2) (layer "F.Cu") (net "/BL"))
 (segment (start 145.6 107.334315) (end 145.834315 107.1) (width 0.2) (layer "F.Cu") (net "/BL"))
 (segment (start 123.770101 123.968) (end 124.929899 123.968) (width 0.2) (layer "F.Cu") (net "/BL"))
 (segment (start 162.929899 123.968) (end 163.75 124.788101) (width 0.2) (layer "F.Cu") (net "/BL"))
 (segment (start 163.75 124.788101) (end 163.75 125.947899) (width 0.2) (layer "F.Cu") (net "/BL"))
 (segment (start 103.95 125.947899) (end 104.770101 126.768) (width 0.2) (layer "F.Cu") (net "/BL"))
 (segment (start 103.95 98.67) (end 103.95 125.947899) (width 0.2) (layer "F.Cu") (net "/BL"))
 (segment (start 145.665685 105.4) (end 145.4 105.4) (width 0.2) (layer "F.Cu") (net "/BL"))
 (segment (start 102 96.72) (end 103.95 98.67) (width 0.2) (layer "F.Cu") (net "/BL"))
 (segment (start 102 96.72) (end 104.35 99.07) (width 0.2) (layer "B.Cu") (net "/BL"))
 (segment (start 131.1305 116.46) (end 129.8305 115.16) (width 0.2) (layer "B.Cu") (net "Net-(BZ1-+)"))
 (segment (start 170.4 102.3) (end 156.24 116.46) (width 0.2) (layer "B.Cu") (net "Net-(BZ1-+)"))
 (segment (start 156.24 116.46) (end 131.1305 116.46) (width 0.2) (layer "B.Cu") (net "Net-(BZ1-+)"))
 (segment (start 102 104.34) (end 103.08 105.42) (width 0.2) (layer "B.Cu") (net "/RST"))
 (segment (start 103.08 105.42) (end 103.15 105.49) (width 0.2) (layer "B.Cu") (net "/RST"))
 (segment (start 168.685685 97.42) (end 172.1 100.834315) (width 0.2) (layer "B.Cu") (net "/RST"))
 (segment (start 128.851172 117.26) (end 127.7555 116.164327) (width 0.2) (layer "B.Cu") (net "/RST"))
 (segment (start 172.1 103.765686) (end 158.605685 117.26) (width 0.2) (layer "B.Cu") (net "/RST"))
 (segment (start 103.08 105.42) (end 111.08 97.42) (width 0.2) (layer "B.Cu") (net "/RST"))
 (segment (start 158.605685 117.26) (end 128.851172 117.26) (width 0.2) (layer "B.Cu") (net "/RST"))
 (segment (start 111.08 97.42) (end 168.685685 97.42) (width 0.2) (layer "B.Cu") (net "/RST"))
 (segment (start 127.7555 116.164327) (end 127.7555 115.832956) (width 0.2) (layer "B.Cu") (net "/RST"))
 (segment (start 172.1 100.834315) (end 172.1 103.765686) (width 0.2) (layer "B.Cu") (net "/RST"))
 (segment (start 131.9055 108.005) (end 129.8305 110.08) (width 0.2) (layer "B.Cu") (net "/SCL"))
 (segment (start 131.209828 98.22) (end 131.9055 98.915673) (width 0.2) (layer "B.Cu") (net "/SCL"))
 (segment (start 131.9055 98.915673) (end 131.9055 108.005) (width 0.2) (layer "B.Cu") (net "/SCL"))
 (segment (start 102 109.42) (end 113.2 98.22) (width 0.2) (layer "B.Cu") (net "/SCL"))
 (segment (start 113.2 98.22) (end 131.209828 98.22) (width 0.2) (layer "B.Cu") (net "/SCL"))
 (segment (start 102 106.88) (end 103.974314 106.88) (width 0.2) (layer "B.Cu") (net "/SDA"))
 (segment (start 144.3205 100.758642) (end 144.3205 99.081358) (width 0.2) (layer "B.Cu") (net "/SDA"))
 (segment (start 131.375514 97.82) (end 132.3055 98.749988) (width 0.2) (layer "B.Cu") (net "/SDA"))
 (segment (start 158.44 116.86) (end 129.016858 116.86) (width 0.2) (layer "B.Cu") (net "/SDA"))
 (segment (start 132.3055 98.749988) (end 132.3055 108.170686) (width 0.2) (layer "B.Cu") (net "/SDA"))
 (segment (start 103.974314 106.88) (end 113.034315 97.82) (width 0.2) (layer "B.Cu") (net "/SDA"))
 (segment (start 128.1555 109.215) (end 129.8305 107.54) (width 0.2) (layer "B.Cu") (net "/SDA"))
 (segment (start 128.1555 115.998642) (end 128.1555 109.215) (width 0.2) (layer "B.Cu") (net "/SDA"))
 (segment (start 169.32 98.62) (end 171.7 101) (width 0.2) (layer "B.Cu") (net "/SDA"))
 (segment (start 136.908456 108.170686) (end 144.3205 100.758642) (width 0.2) (layer "B.Cu") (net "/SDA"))
 (segment (start 144.3205 99.081358) (end 144.781858 98.62) (width 0.2) (layer "B.Cu") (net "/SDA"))
 (segment (start 132.3055 108.170686) (end 136.908456 108.170686) (width 0.2) (layer "B.Cu") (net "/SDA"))
 (segment (start 144.781858 98.62) (end 169.32 98.62) (width 0.2) (layer "B.Cu") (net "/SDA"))
 (segment (start 129.016858 116.86) (end 128.1555 115.998642) (width 0.2) (layer "B.Cu") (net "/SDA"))
 (segment (start 113.034315 97.82) (end 131.375514 97.82) (width 0.2) (layer "B.Cu") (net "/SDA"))
 (segment (start 171.7 101) (end 171.7 103.6) (width 0.2) (layer "B.Cu") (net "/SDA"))
 (segment (start 171.7 103.6) (end 158.44 116.86) (width 0.2) (layer "B.Cu") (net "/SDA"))
 (segment (start 131.044142 98.62) (end 131.5055 99.081358) (width 0.2) (layer "B.Cu") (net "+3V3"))
 (segment (start 131.5055 99.081358) (end 131.5055 103.325) (width 0.2) (layer "B.Cu") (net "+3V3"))
 (segment (start 120.96 113.5) (end 120.96 106.276858) (width 0.2) (layer "B.Cu") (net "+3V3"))
 (segment (start 102 111.96) (end 115.34 98.62) (width 0.2) (layer "B.Cu") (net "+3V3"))
 (segment (start 131.044142 98.62) (end 128.616858 98.62) (width 0.2) (layer "B.Cu") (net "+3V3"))
 (segment (start 131.5055 103.325) (end 129.8305 105) (width 0.2) (layer "B.Cu") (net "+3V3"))
 (segment (start 115.34 98.62) (end 131.044142 98.62) (width 0.2) (layer "B.Cu") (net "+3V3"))
 (segment (start 128.616858 98.62) (end 120.96 106.276858) (width 0.2) (layer "B.Cu") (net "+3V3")))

